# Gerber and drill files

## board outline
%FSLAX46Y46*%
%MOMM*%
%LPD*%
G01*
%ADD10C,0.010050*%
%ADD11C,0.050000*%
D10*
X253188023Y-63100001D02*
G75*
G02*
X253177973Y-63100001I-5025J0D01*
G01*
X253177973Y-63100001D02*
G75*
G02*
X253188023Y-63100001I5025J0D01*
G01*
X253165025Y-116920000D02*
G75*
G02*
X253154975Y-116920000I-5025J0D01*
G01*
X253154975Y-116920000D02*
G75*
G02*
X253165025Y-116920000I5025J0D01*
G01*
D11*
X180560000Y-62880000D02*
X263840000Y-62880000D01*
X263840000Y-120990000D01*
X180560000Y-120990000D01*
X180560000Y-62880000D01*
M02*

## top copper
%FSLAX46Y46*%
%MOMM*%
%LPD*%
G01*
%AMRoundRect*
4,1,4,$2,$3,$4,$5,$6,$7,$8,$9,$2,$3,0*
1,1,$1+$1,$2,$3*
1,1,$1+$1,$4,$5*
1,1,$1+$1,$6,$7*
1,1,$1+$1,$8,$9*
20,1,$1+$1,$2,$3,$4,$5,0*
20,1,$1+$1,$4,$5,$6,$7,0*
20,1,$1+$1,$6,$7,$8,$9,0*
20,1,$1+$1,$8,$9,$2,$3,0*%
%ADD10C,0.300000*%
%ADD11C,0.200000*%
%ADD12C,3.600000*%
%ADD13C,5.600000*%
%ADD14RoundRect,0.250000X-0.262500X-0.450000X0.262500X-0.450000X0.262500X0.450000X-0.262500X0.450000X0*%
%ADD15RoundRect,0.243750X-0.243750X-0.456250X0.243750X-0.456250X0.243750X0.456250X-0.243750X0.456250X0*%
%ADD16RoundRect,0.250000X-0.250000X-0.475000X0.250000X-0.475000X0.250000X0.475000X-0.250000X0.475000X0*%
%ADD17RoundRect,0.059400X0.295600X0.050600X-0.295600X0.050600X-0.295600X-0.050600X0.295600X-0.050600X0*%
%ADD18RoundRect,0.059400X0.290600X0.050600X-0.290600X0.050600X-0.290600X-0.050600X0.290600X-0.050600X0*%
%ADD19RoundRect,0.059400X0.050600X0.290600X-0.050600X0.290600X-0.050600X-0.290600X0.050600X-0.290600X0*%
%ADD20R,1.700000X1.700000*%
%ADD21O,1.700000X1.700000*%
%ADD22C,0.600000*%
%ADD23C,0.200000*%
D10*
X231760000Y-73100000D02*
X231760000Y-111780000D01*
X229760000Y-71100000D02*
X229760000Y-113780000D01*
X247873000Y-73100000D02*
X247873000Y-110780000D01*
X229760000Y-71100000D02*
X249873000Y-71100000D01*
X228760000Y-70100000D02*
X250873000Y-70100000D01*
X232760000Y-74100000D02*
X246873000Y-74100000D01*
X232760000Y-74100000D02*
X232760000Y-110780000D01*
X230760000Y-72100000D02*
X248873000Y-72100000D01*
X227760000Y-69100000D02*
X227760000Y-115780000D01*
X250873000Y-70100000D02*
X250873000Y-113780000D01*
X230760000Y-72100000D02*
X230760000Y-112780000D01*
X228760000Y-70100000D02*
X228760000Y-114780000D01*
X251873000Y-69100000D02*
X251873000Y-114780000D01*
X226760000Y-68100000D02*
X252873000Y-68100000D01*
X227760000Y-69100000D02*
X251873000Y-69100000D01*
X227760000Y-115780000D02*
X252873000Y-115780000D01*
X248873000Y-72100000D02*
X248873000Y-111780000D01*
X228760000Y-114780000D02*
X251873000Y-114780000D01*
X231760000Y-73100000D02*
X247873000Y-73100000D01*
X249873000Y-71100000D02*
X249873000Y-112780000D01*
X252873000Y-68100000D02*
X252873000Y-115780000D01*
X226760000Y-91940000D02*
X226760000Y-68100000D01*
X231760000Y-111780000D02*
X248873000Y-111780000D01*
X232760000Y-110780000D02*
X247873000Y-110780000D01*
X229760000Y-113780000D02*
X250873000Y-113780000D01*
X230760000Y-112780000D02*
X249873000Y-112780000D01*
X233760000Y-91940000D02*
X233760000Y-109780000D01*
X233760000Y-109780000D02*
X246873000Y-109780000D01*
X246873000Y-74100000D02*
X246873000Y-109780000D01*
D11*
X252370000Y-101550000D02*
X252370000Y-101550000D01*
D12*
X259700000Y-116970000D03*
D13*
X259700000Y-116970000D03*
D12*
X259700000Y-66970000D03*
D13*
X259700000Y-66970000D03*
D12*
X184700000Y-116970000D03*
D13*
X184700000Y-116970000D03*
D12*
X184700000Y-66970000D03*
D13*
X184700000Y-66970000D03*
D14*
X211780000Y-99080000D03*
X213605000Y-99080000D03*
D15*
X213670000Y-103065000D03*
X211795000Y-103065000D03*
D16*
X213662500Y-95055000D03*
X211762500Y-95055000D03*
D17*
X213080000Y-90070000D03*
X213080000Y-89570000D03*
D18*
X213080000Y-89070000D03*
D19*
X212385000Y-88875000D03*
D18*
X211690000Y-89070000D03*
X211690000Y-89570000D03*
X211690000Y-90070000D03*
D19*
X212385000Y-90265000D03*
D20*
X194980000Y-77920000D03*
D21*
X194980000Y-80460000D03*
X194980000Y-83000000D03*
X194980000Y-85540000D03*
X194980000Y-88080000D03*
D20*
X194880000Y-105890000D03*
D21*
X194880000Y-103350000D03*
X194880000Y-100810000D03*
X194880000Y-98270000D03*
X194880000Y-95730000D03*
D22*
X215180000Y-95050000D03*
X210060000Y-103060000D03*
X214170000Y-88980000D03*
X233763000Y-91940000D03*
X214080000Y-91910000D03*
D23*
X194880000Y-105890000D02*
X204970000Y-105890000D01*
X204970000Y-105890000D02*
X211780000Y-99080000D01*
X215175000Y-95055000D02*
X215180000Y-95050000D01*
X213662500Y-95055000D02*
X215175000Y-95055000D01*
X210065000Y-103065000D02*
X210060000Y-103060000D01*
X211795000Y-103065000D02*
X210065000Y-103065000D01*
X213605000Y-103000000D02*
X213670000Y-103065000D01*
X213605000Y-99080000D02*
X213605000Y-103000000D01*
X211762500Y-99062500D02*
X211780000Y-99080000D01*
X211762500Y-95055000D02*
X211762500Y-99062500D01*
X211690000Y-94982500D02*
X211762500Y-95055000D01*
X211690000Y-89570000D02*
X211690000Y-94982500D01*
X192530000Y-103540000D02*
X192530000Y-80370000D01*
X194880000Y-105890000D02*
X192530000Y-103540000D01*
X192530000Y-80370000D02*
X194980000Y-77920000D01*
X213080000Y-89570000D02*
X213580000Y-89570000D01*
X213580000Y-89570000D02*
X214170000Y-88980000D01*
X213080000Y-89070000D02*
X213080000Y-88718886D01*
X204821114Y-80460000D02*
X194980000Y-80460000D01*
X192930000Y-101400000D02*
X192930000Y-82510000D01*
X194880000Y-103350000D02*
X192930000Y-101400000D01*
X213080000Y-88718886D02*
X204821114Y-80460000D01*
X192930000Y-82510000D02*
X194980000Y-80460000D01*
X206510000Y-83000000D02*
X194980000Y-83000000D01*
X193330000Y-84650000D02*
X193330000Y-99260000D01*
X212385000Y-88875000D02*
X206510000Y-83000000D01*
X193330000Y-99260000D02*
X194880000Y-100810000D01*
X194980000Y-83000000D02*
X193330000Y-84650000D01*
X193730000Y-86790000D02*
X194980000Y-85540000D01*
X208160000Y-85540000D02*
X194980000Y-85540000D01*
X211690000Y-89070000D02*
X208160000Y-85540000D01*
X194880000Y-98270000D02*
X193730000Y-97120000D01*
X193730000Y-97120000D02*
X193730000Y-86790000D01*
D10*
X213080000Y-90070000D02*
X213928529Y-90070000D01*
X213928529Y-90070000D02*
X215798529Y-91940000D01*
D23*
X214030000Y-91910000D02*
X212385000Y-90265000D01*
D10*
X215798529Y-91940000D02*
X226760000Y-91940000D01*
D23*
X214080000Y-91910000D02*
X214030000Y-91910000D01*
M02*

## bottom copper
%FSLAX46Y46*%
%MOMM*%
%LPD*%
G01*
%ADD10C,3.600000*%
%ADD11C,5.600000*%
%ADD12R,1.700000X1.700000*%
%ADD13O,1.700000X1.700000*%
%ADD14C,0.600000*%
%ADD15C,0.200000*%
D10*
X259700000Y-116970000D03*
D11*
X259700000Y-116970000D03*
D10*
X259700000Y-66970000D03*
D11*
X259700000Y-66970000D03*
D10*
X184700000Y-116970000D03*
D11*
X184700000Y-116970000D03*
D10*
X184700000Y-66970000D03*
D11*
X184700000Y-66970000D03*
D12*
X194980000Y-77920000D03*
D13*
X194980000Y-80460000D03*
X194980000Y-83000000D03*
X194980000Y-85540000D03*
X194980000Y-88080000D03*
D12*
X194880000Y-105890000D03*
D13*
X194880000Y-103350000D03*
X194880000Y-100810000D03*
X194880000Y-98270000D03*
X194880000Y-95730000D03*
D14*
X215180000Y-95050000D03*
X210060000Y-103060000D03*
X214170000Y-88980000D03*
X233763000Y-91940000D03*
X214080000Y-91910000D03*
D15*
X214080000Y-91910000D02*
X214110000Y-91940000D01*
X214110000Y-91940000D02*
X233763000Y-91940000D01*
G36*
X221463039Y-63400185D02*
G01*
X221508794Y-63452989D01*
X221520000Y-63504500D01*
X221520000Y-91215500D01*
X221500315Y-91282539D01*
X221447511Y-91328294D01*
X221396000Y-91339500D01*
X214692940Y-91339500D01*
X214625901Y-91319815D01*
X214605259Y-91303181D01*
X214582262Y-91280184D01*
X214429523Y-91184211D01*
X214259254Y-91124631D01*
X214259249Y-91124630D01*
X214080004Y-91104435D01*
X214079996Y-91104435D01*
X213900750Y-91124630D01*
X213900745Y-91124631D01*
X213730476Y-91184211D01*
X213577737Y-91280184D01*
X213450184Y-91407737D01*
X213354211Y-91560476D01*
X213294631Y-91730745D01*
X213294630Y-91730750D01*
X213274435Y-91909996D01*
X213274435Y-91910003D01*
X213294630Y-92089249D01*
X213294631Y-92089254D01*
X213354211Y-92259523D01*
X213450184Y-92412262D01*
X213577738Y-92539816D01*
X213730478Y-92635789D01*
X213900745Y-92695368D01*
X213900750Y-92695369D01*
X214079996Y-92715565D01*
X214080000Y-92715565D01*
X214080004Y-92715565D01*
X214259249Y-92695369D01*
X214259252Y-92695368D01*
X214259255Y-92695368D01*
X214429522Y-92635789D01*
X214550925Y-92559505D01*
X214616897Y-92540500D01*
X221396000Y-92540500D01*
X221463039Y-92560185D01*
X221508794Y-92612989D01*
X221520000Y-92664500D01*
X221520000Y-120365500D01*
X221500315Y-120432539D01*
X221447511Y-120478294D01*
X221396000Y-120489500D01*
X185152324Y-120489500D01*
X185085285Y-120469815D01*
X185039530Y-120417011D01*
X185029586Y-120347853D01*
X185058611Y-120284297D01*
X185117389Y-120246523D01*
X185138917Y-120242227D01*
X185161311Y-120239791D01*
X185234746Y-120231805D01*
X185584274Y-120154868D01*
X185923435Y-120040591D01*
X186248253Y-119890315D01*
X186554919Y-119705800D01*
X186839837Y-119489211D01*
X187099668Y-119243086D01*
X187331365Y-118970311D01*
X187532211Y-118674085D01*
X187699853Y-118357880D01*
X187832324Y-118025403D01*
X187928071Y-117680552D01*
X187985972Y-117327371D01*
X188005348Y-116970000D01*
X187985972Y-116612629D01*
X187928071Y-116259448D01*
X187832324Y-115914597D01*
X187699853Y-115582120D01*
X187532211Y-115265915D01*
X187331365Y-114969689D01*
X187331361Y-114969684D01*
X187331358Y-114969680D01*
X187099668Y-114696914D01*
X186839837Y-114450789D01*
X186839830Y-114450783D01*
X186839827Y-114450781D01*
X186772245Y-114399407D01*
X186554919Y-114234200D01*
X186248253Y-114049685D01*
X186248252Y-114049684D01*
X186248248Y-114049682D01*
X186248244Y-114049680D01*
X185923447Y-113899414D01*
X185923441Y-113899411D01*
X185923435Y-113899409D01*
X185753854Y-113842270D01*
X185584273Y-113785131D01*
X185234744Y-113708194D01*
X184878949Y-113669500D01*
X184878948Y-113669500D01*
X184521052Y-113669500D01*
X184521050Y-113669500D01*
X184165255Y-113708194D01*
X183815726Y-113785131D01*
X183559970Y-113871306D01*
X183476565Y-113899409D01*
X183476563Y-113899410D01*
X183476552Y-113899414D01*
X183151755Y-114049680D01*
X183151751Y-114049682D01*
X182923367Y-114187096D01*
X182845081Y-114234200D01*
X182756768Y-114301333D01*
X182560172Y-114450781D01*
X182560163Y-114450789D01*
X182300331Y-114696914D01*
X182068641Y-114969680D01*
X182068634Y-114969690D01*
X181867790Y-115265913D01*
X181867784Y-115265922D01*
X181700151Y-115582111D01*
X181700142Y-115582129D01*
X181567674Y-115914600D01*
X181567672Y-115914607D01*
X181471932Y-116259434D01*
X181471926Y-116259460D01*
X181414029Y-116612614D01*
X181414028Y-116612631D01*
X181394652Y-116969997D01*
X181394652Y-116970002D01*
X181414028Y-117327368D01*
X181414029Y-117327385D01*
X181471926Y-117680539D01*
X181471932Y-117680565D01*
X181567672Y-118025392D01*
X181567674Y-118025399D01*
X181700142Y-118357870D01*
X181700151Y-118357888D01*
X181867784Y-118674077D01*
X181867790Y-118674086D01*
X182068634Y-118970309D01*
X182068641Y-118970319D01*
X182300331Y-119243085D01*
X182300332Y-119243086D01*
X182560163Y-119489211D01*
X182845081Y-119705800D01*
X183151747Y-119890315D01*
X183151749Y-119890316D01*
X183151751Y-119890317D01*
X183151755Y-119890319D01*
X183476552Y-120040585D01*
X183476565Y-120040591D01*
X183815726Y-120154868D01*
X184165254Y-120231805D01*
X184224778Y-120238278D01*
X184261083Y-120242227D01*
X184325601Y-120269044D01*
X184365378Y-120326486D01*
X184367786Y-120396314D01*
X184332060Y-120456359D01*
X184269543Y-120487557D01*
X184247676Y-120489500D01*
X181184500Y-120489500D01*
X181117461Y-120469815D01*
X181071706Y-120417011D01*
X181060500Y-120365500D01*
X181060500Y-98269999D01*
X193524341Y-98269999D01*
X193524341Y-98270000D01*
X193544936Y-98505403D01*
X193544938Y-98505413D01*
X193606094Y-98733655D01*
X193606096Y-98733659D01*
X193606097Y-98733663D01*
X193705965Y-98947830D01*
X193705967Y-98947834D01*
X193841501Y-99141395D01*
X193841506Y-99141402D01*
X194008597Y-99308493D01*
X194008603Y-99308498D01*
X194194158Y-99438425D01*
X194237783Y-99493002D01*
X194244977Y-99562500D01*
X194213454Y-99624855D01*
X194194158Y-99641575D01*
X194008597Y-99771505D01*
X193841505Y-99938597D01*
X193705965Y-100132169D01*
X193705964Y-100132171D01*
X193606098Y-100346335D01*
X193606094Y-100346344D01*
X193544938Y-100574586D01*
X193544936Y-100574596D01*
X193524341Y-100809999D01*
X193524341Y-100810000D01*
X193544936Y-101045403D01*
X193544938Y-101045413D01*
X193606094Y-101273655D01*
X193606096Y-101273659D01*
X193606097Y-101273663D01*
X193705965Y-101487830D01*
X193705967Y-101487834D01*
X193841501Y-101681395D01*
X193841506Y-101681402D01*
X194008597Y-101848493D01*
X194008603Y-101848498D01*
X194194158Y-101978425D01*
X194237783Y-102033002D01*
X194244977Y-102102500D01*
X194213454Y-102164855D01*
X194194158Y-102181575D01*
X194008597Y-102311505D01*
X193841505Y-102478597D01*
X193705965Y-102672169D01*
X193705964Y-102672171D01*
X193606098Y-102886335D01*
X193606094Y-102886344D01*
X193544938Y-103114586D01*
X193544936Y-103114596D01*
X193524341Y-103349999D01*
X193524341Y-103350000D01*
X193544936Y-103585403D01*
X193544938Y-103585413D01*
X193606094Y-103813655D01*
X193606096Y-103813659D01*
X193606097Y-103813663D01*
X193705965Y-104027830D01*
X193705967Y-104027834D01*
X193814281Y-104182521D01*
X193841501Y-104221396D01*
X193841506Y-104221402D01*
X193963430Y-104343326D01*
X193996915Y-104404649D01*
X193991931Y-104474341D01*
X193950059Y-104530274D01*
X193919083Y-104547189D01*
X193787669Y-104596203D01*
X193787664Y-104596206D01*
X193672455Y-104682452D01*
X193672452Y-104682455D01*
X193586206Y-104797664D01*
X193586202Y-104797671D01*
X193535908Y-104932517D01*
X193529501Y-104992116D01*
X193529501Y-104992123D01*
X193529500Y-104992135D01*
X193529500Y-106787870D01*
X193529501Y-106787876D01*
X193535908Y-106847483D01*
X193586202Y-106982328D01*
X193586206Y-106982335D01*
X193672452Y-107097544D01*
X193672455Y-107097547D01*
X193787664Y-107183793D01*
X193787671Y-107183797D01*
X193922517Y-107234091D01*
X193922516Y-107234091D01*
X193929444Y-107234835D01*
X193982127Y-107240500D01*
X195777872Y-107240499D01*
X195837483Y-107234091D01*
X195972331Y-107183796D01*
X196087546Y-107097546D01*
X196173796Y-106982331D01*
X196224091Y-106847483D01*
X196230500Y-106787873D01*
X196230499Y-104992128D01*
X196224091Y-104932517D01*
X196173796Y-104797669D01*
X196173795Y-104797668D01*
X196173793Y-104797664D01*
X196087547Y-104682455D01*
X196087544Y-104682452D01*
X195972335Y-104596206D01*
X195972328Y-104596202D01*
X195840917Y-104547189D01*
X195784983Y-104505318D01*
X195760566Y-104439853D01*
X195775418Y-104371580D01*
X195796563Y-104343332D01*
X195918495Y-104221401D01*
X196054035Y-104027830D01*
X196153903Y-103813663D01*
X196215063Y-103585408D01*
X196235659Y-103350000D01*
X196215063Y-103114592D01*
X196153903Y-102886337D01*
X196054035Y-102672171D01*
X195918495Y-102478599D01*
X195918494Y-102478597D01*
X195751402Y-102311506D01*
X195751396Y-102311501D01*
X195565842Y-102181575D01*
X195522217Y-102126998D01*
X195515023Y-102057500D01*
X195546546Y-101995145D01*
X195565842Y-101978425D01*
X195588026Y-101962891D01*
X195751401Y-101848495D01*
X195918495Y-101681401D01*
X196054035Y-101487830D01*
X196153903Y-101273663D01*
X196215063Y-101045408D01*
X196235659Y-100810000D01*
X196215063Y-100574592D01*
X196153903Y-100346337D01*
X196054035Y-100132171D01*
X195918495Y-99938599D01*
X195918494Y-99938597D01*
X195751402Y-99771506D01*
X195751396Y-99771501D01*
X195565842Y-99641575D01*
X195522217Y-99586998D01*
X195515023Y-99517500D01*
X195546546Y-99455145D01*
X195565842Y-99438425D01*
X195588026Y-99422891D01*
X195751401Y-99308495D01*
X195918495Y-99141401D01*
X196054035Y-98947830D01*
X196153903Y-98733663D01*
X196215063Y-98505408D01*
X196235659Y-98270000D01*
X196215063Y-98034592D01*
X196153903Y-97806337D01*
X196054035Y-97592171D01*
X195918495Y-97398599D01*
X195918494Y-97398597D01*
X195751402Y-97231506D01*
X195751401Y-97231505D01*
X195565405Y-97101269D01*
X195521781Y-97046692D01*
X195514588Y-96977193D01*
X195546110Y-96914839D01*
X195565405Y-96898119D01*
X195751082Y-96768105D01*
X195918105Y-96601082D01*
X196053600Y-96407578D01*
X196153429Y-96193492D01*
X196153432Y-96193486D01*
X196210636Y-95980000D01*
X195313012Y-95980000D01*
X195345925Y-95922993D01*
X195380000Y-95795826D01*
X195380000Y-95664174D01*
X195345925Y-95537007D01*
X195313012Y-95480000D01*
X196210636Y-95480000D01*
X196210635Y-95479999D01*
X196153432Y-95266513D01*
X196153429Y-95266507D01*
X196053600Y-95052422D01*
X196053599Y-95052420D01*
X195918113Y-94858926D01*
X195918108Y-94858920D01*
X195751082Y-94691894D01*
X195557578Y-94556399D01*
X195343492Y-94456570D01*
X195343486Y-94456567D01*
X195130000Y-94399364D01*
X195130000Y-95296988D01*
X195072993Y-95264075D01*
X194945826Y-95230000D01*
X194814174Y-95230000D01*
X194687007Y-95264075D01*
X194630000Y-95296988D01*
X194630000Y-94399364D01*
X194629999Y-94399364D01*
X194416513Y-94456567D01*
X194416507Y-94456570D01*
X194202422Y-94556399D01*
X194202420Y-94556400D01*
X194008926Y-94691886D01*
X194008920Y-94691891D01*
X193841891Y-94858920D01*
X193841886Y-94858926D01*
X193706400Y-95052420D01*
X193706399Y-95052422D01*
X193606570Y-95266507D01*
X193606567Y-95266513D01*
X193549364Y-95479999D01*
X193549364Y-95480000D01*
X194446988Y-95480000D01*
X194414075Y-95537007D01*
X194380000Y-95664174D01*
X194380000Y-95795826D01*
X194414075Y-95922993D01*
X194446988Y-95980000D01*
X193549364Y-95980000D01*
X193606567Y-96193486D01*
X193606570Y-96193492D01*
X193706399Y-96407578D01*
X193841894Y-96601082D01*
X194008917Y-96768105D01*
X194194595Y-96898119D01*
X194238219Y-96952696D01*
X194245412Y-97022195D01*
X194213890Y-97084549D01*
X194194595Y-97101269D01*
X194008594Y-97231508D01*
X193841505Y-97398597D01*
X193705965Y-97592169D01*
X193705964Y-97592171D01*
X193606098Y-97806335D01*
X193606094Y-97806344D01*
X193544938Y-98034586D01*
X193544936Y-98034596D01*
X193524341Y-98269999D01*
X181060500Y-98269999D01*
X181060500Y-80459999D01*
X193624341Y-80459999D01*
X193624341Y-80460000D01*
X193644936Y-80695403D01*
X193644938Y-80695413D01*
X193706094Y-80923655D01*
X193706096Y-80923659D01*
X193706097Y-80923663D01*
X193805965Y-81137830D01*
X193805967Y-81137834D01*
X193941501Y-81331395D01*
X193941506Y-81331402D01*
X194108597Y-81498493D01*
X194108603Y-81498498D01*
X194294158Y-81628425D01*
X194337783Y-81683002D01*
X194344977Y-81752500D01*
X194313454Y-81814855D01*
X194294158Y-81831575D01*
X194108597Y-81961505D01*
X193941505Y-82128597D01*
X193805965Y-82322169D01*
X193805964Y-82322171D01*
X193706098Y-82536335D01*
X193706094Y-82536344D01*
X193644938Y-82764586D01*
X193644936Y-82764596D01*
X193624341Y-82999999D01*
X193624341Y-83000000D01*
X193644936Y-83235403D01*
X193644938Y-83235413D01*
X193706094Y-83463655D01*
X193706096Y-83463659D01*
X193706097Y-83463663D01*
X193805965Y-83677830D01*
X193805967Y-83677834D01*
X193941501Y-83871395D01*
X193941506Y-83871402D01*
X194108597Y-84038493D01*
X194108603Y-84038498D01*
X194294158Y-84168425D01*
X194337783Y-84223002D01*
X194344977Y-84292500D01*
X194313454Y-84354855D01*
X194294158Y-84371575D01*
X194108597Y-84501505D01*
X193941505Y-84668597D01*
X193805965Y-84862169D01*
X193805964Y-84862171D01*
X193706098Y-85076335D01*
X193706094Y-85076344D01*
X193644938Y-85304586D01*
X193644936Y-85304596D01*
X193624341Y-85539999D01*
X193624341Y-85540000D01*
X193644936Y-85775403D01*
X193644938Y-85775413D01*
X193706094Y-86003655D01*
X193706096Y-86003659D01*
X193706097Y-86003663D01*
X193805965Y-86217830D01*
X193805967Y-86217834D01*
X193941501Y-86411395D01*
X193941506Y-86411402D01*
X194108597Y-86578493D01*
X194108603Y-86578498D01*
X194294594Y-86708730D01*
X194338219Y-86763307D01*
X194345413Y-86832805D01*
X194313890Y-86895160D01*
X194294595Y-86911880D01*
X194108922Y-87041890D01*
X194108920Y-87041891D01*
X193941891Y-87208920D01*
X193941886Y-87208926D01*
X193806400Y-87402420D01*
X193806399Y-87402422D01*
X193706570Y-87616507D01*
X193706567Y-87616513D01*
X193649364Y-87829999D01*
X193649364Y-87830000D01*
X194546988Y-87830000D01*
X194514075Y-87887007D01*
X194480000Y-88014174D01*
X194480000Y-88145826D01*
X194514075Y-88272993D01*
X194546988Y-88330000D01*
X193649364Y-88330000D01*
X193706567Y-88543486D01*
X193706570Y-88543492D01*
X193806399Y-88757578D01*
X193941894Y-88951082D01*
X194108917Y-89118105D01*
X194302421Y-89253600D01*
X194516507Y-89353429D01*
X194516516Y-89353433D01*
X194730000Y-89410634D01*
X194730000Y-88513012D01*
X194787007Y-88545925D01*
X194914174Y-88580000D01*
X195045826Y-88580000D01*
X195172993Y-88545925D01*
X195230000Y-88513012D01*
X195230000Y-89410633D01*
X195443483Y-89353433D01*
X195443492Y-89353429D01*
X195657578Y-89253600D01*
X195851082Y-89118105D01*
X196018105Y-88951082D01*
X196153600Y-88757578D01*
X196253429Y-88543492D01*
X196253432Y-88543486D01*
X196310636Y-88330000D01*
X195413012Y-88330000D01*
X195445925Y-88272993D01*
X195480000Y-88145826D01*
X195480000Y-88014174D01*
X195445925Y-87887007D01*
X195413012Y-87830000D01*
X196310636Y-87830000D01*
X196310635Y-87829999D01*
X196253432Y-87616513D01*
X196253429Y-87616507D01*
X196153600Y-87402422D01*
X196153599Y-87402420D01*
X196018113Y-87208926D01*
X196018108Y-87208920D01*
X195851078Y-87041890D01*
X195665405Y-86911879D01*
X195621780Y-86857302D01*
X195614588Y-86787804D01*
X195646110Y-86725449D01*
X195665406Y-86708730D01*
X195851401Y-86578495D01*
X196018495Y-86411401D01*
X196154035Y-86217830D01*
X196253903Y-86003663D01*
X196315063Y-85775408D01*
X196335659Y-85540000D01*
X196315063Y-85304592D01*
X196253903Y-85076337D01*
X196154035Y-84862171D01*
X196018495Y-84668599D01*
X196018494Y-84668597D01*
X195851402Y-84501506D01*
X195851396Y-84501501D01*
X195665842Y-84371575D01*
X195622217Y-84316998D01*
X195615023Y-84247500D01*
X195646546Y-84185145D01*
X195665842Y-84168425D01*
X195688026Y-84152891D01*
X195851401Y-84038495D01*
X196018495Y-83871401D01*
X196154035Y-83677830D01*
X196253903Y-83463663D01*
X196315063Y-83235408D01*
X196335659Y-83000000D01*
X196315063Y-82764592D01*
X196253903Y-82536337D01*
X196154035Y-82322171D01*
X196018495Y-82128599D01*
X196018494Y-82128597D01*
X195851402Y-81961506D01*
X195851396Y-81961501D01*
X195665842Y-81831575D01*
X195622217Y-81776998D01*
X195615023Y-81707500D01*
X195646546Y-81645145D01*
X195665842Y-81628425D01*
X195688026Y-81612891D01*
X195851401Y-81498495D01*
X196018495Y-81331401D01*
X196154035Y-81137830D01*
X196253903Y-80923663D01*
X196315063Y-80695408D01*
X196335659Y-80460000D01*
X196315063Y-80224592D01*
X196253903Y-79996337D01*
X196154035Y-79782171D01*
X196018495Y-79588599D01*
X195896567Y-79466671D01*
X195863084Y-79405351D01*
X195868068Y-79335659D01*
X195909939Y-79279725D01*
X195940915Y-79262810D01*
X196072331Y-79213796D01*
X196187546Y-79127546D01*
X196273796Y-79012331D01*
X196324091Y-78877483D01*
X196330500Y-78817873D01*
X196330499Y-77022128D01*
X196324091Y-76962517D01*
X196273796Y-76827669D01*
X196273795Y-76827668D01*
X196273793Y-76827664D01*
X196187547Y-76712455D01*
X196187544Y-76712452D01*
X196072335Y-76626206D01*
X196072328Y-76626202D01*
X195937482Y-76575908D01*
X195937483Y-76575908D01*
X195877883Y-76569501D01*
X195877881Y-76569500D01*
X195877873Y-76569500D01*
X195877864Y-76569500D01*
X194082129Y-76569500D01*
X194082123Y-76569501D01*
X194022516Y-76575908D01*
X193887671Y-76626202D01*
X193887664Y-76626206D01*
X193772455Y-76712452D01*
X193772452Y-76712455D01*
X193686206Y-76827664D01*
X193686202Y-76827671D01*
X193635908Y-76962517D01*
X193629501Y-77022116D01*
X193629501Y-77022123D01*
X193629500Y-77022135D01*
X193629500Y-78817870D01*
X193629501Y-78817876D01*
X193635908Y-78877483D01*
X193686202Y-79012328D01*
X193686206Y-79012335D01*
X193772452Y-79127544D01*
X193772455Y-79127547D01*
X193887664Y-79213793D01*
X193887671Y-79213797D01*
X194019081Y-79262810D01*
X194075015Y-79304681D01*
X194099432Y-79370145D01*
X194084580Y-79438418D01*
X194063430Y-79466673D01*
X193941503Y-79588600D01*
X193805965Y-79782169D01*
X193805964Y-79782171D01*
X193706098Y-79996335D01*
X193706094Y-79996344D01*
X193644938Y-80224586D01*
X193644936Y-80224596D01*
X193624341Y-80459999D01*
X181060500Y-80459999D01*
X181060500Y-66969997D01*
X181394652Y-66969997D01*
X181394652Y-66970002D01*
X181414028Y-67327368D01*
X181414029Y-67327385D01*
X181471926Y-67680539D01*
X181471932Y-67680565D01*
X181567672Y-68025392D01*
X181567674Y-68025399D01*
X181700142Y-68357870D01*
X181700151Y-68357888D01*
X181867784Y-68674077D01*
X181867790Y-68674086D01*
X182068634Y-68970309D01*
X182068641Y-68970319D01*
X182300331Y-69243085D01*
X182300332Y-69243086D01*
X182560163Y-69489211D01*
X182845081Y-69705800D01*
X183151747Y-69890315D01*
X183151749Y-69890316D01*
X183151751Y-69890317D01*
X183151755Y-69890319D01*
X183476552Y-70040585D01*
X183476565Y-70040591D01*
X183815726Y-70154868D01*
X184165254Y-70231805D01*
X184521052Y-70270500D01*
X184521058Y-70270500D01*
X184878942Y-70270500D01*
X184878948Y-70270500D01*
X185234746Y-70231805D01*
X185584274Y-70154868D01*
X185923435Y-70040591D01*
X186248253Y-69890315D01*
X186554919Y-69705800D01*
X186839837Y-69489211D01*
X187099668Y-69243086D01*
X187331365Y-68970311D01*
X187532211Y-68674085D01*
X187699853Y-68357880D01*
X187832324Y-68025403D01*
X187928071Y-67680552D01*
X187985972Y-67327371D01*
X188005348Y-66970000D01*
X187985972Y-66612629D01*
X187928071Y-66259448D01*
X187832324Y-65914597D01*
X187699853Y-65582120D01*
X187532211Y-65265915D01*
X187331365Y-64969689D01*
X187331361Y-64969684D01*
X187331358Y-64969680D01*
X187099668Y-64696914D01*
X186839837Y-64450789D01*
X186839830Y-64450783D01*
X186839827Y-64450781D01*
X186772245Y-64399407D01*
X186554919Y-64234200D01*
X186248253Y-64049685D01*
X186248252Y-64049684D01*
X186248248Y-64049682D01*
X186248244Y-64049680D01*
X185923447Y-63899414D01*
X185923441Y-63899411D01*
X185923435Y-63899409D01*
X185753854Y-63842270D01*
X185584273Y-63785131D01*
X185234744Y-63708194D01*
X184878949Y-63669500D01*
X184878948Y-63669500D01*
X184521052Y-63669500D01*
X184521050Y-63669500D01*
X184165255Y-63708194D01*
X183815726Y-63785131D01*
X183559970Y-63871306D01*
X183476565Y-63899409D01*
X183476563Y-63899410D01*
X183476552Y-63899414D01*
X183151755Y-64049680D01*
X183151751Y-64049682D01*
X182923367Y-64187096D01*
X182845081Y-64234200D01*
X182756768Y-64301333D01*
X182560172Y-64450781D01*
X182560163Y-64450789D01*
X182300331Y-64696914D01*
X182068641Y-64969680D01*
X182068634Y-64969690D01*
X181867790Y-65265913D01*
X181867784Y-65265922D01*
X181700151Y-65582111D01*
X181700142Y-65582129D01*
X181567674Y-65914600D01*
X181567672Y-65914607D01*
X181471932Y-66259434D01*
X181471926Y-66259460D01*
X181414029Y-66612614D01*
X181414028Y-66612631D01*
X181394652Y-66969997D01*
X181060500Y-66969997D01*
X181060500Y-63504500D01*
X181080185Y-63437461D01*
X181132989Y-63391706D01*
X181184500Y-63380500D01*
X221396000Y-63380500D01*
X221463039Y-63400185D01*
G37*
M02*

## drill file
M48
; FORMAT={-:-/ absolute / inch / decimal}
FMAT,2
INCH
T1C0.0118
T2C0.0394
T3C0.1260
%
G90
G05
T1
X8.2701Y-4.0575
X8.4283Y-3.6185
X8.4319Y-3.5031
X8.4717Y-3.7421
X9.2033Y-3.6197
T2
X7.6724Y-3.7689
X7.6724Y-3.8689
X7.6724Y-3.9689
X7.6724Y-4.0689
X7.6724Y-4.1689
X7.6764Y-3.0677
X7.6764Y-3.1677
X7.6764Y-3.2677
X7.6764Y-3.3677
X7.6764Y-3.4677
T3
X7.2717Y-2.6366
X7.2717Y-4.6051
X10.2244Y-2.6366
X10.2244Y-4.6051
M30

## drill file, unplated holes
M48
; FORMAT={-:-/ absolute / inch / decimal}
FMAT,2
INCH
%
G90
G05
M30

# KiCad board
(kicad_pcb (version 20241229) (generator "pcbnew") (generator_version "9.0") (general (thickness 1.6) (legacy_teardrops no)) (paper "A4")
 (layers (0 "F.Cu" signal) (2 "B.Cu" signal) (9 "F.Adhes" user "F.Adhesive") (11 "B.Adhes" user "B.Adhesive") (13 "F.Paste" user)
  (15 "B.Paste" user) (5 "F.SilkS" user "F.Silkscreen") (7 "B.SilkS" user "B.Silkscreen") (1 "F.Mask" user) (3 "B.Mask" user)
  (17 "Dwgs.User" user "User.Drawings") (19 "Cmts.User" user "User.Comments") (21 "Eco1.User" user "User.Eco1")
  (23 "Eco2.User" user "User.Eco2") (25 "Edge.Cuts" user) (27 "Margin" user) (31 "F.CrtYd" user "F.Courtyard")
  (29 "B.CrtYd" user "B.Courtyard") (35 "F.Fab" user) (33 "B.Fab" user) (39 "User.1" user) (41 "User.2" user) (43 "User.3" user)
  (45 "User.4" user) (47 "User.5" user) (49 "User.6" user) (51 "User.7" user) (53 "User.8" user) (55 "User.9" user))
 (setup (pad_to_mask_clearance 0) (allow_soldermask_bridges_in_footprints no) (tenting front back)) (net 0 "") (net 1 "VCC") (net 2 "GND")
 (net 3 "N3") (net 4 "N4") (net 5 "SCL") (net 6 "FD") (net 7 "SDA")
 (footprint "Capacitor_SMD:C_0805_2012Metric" (layer "F.Cu") (at 212.7125 95.055)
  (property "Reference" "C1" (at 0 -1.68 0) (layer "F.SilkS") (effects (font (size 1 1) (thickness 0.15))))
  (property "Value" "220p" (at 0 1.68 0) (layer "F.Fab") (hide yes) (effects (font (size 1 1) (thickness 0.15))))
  (pad "1" smd roundrect (at -0.95 0) (size 1 1.45) (layers "F.Cu" "F.Mask" "F.Paste") (roundrect_rratio 0.25) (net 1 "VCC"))
  (pad "2" smd roundrect (at 0.95 0) (size 1 1.45) (layers "F.Cu" "F.Mask" "F.Paste") (roundrect_rratio 0.25) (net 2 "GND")))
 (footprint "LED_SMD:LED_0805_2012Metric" (layer "F.Cu") (at 212.7325 103.065)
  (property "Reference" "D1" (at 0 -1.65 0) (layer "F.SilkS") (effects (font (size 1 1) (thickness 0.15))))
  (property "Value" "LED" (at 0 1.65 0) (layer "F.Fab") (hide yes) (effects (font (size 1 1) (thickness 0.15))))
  (pad "1" smd roundrect (at -0.9375 0) (size 0.975 1.4) (layers "F.Cu" "F.Mask" "F.Paste") (roundrect_rratio 0.25) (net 2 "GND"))
  (pad "2" smd roundrect (at 0.9375 0) (size 0.975 1.4) (layers "F.Cu" "F.Mask" "F.Paste") (roundrect_rratio 0.25) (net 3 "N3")))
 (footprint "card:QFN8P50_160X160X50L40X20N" (layer "F.Cu") (at 212.385 89.57 180)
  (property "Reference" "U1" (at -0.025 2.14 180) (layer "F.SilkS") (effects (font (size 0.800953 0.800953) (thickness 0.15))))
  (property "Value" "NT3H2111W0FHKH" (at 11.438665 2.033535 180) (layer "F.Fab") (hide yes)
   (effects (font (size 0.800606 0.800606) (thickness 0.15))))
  (pad "1" smd roundrect (at -0.695 -0.5 180) (size 0.71 0.22) (layers "F.Cu" "F.Mask" "F.Paste") (roundrect_rratio 0.27) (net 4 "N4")
   (solder_mask_margin 0.102))
  (pad "2" smd roundrect (at -0.695 0 180) (size 0.71 0.22) (layers "F.Cu" "F.Mask" "F.Paste") (roundrect_rratio 0.27) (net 2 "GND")
   (solder_mask_margin 0.102))
  (pad "3" smd roundrect (at -0.695 0.5 180) (size 0.7 0.22) (layers "F.Cu" "F.Mask" "F.Paste") (roundrect_rratio 0.27) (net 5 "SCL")
   (solder_mask_margin 0.102))
  (pad "4" smd roundrect (at 0 0.695 180) (size 0.22 0.7) (layers "F.Cu" "F.Mask" "F.Paste") (roundrect_rratio 0.27) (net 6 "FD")
   (solder_mask_margin 0.102))
  (pad "5" smd roundrect (at 0.695 0.5 180) (size 0.7 0.22) (layers "F.Cu" "F.Mask" "F.Paste") (roundrect_rratio 0.27) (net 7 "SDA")
   (solder_mask_margin 0.102))
  (pad "6" smd roundrect (at 0.695 0 180) (size 0.7 0.22) (layers "F.Cu" "F.Mask" "F.Paste") (roundrect_rratio 0.27) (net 1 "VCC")
   (solder_mask_margin 0.102))
  (pad "7" smd roundrect (at 0.695 -0.5 180) (size 0.7 0.22) (layers "F.Cu" "F.Mask" "F.Paste") (roundrect_rratio 0.27) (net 1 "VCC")
   (solder_mask_margin 0.102))
  (pad "8" smd roundrect (at 0 -0.695 180) (size 0.22 0.7) (layers "F.Cu" "F.Mask" "F.Paste") (roundrect_rratio 0.27) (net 4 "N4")
   (solder_mask_margin 0.102)))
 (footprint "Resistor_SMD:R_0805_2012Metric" (layer "F.Cu") (at 212.6925 99.08)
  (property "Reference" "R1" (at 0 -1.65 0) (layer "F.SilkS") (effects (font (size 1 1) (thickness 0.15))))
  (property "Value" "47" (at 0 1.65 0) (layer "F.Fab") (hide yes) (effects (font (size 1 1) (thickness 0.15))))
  (pad "1" smd roundrect (at -0.9125 0) (size 1.025 1.4) (layers "F.Cu" "F.Mask" "F.Paste") (roundrect_rratio 0.243902) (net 1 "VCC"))
  (pad "2" smd roundrect (at 0.9125 0) (size 1.025 1.4) (layers "F.Cu" "F.Mask" "F.Paste") (roundrect_rratio 0.243902) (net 3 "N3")))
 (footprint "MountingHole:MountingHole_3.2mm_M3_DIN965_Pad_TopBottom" (layer "F.Cu") (at 259.7 66.97)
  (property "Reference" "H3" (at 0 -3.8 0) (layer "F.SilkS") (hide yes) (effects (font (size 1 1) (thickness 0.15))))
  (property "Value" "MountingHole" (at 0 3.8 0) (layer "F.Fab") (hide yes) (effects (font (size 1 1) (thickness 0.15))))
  (pad "1" thru_hole circle (at 0 0) (size 3.6 3.6) (drill 3.2) (layers "*.Cu" "*.Mask") (remove_unused_layers no))
  (pad "1" connect circle (at 0 0) (size 5.6 5.6) (layers "F.Cu" "F.Mask"))
  (pad "1" connect circle (at 0 0) (size 5.6 5.6) (layers "B.Cu" "B.Mask")))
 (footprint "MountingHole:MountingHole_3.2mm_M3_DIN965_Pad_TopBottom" (layer "F.Cu") (at 184.7 116.97)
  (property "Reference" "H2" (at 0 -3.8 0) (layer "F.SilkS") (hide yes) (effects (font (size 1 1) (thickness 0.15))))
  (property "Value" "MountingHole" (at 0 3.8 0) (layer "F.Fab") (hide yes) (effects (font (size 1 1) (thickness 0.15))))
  (pad "1" thru_hole circle (at 0 0) (size 3.6 3.6) (drill 3.2) (layers "*.Cu" "*.Mask") (remove_unused_layers no))
  (pad "1" connect circle (at 0 0) (size 5.6 5.6) (layers "F.Cu" "F.Mask"))
  (pad "1" connect circle (at 0 0) (size 5.6 5.6) (layers "B.Cu" "B.Mask")))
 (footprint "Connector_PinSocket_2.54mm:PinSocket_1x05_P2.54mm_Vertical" (layer "F.Cu") (at 194.98 77.92)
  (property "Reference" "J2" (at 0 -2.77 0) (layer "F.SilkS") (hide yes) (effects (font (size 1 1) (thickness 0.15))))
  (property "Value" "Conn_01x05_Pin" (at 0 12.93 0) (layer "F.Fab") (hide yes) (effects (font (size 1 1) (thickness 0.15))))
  (pad "1" thru_hole rect (at 0 0) (size 1.7 1.7) (drill 1) (layers "*.Cu" "*.Mask") (remove_unused_layers no) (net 1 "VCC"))
  (pad "2" thru_hole oval (at 0 2.54) (size 1.7 1.7) (drill 1) (layers "*.Cu" "*.Mask") (remove_unused_layers no) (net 5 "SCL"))
  (pad "3" thru_hole oval (at 0 5.08) (size 1.7 1.7) (drill 1) (layers "*.Cu" "*.Mask") (remove_unused_layers no) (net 6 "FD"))
  (pad "4" thru_hole oval (at 0 7.62) (size 1.7 1.7) (drill 1) (layers "*.Cu" "*.Mask") (remove_unused_layers no) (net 7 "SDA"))
  (pad "5" thru_hole oval (at 0 10.16) (size 1.7 1.7) (drill 1) (layers "*.Cu" "*.Mask") (remove_unused_layers no) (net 2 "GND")))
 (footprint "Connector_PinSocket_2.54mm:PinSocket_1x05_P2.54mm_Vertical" (layer "F.Cu") (at 194.88 105.89 180)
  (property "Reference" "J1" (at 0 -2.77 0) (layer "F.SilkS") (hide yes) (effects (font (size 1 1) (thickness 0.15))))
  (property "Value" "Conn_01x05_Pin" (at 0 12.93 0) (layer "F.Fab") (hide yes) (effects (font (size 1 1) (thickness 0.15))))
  (pad "1" thru_hole rect (at 0 0 180) (size 1.7 1.7) (drill 1) (layers "*.Cu" "*.Mask") (remove_unused_layers no) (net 1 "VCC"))
  (pad "2" thru_hole oval (at 0 2.54 180) (size 1.7 1.7) (drill 1) (layers "*.Cu" "*.Mask") (remove_unused_layers no) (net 5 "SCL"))
  (pad "3" thru_hole oval (at 0 5.08 180) (size 1.7 1.7) (drill 1) (layers "*.Cu" "*.Mask") (remove_unused_layers no) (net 6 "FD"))
  (pad "4" thru_hole oval (at 0 7.62 180) (size 1.7 1.7) (drill 1) (layers "*.Cu" "*.Mask") (remove_unused_layers no) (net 7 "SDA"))
  (pad "5" thru_hole oval (at 0 10.16 180) (size 1.7 1.7) (drill 1) (layers "*.Cu" "*.Mask") (remove_unused_layers no) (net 2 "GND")))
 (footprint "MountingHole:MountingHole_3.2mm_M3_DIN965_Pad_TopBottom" (layer "F.Cu") (at 184.7 66.97)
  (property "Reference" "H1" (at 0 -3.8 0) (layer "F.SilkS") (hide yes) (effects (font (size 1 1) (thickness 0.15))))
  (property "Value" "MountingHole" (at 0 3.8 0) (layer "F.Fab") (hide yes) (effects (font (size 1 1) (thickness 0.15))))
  (pad "1" thru_hole circle (at 0 0) (size 3.6 3.6) (drill 3.2) (layers "*.Cu" "*.Mask") (remove_unused_layers no))
  (pad "1" connect circle (at 0 0) (size 5.6 5.6) (layers "F.Cu" "F.Mask"))
  (pad "1" connect circle (at 0 0) (size 5.6 5.6) (layers "B.Cu" "B.Mask")))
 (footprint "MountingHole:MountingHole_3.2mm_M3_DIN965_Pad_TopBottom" (layer "F.Cu") (at 259.7 116.97)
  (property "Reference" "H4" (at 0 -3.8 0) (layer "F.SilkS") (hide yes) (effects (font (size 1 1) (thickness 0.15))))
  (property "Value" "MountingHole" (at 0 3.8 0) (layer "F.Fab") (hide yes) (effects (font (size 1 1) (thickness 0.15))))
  (pad "1" thru_hole circle (at 0 0) (size 3.6 3.6) (drill 3.2) (layers "*.Cu" "*.Mask") (remove_unused_layers no))
  (pad "1" connect circle (at 0 0) (size 5.6 5.6) (layers "F.Cu" "F.Mask"))
  (pad "1" connect circle (at 0 0) (size 5.6 5.6) (layers "B.Cu" "B.Mask")))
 (gr_line (start 231.76 73.1) (end 231.76 111.78) (stroke (width 0.3) (type default)) (layer "F.Cu") (net 4))
 (gr_line (start 229.76 71.1) (end 229.76 113.78) (stroke (width 0.3) (type default)) (layer "F.Cu") (net 4))
 (gr_line (start 247.873 73.1) (end 247.873 110.78) (stroke (width 0.3) (type default)) (layer "F.Cu") (net 4))
 (gr_line (start 229.76 71.1) (end 249.873 71.1) (stroke (width 0.3) (type default)) (layer "F.Cu") (net 4))
 (gr_line (start 228.76 70.1) (end 250.873 70.1) (stroke (width 0.3) (type default)) (layer "F.Cu") (net 4))
 (gr_line (start 232.76 74.1) (end 246.873 74.1) (stroke (width 0.3) (type default)) (layer "F.Cu") (net 4))
 (gr_line (start 232.76 74.1) (end 232.76 110.78) (stroke (width 0.3) (type default)) (layer "F.Cu") (net 4))
 (gr_line (start 230.76 72.1) (end 248.873 72.1) (stroke (width 0.3) (type default)) (layer "F.Cu") (net 4))
 (gr_line (start 227.76 69.1) (end 227.76 115.78) (stroke (width 0.3) (type default)) (layer "F.Cu") (net 4))
 (gr_line (start 250.873 70.1) (end 250.873 113.78) (stroke (width 0.3) (type default)) (layer "F.Cu") (net 4))
 (gr_line (start 230.76 72.1) (end 230.76 112.78) (stroke (width 0.3) (type default)) (layer "F.Cu") (net 4))
 (gr_line (start 228.76 70.1) (end 228.76 114.78) (stroke (width 0.3) (type default)) (layer "F.Cu") (net 4))
 (gr_line (start 251.873 69.1) (end 251.873 114.78) (stroke (width 0.3) (type default)) (layer "F.Cu") (net 4))
 (gr_line (start 226.76 68.1) (end 252.873 68.1) (stroke (width 0.3) (type default)) (layer "F.Cu") (net 4))
 (gr_line (start 227.76 69.1) (end 251.873 69.1) (stroke (width 0.3) (type default)) (layer "F.Cu") (net 4))
 (gr_line (start 227.76 115.78) (end 252.873 115.78) (stroke (width 0.3) (type default)) (layer "F.Cu") (net 4))
 (gr_line (start 248.873 72.1) (end 248.873 111.78) (stroke (width 0.3) (type default)) (layer "F.Cu") (net 4))
 (gr_line (start 228.76 114.78) (end 251.873 114.78) (stroke (width 0.3) (type default)) (layer "F.Cu") (net 4))
 (gr_line (start 231.76 73.1) (end 247.873 73.1) (stroke (width 0.3) (type default)) (layer "F.Cu") (net 4))
 (gr_line (start 249.873 71.1) (end 249.873 112.78) (stroke (width 0.3) (type default)) (layer "F.Cu") (net 4))
 (gr_line (start 252.873 68.1) (end 252.873 115.78) (stroke (width 0.3) (type default)) (layer "F.Cu") (net 4))
 (gr_line (start 226.76 91.94) (end 226.76 68.1) (stroke (width 0.3) (type default)) (layer "F.Cu") (net 4))
 (gr_line (start 231.76 111.78) (end 248.873 111.78) (stroke (width 0.3) (type default)) (layer "F.Cu") (net 4))
 (gr_line (start 232.76 110.78) (end 247.873 110.78) (stroke (width 0.3) (type default)) (layer "F.Cu") (net 4))
 (gr_line (start 229.76 113.78) (end 250.873 113.78) (stroke (width 0.3) (type default)) (layer "F.Cu") (net 4))
 (gr_line (start 230.76 112.78) (end 249.873 112.78) (stroke (width 0.3) (type default)) (layer "F.Cu") (net 4))
 (gr_line (start 233.76 91.94) (end 233.76 109.78) (stroke (width 0.3) (type default)) (layer "F.Cu") (net 4))
 (gr_line (start 233.76 109.78) (end 246.873 109.78) (stroke (width 0.3) (type default)) (layer "F.Cu") (net 4))
 (gr_line (start 246.873 74.1) (end 246.873 109.78) (stroke (width 0.3) (type default)) (layer "F.Cu") (net 4))
 (gr_line (start 252.37 101.55) (end 252.37 101.55) (stroke (width 0.2) (type default)) (layer "F.Cu"))
 (gr_circle (center 253.182998 63.100001) (end 253.192998 63.100001) (stroke (width 0.0001) (type default)) (fill yes) (layer "Edge.Cuts"))
 (gr_circle (center 253.16 116.92) (end 253.17 116.92) (stroke (width 0.0001) (type default)) (fill yes) (layer "Edge.Cuts"))
 (gr_rect (start 180.56 62.88) (end 263.84 120.99) (stroke (width 0.05) (type default)) (fill no) (layer "Edge.Cuts"))
 (segment (start 211.69 89.57) (end 211.69 94.9825) (width 0.2) (layer "F.Cu") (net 1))
 (segment (start 211.7625 99.0625) (end 211.78 99.08) (width 0.2) (layer "F.Cu") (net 1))
 (segment (start 211.69 94.9825) (end 211.7625 95.055) (width 0.2) (layer "F.Cu") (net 1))
 (segment (start 194.88 105.89) (end 204.97 105.89) (width 0.2) (layer "F.Cu") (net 1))
 (segment (start 192.53 103.54) (end 192.53 80.37) (width 0.2) (layer "F.Cu") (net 1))
 (segment (start 194.88 105.89) (end 192.53 103.54) (width 0.2) (layer "F.Cu") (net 1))
 (segment (start 204.97 105.89) (end 211.78 99.08) (width 0.2) (layer "F.Cu") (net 1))
 (segment (start 192.53 80.37) (end 194.98 77.92) (width 0.2) (layer "F.Cu") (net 1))
 (segment (start 211.7625 95.055) (end 211.7625 99.0625) (width 0.2) (layer "F.Cu") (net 1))
 (segment (start 213.6625 95.055) (end 215.175 95.055) (width 0.2) (layer "F.Cu") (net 2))
 (segment (start 213.08 89.57) (end 213.58 89.57) (width 0.2) (layer "F.Cu") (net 2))
 (segment (start 210.065 103.065) (end 210.06 103.06) (width 0.2) (layer "F.Cu") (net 2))
 (segment (start 213.58 89.57) (end 214.17 88.98) (width 0.2) (layer "F.Cu") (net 2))
 (segment (start 211.795 103.065) (end 210.065 103.065) (width 0.2) (layer "F.Cu") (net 2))
 (segment (start 215.175 95.055) (end 215.18 95.05) (width 0.2) (layer "F.Cu") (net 2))
 (via (at 214.17 88.98) (size 0.6) (drill 0.3) (layers "F.Cu" "B.Cu") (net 2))
 (via (at 210.06 103.06) (size 0.6) (drill 0.3) (layers "F.Cu" "B.Cu") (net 2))
 (via (at 215.18 95.05) (size 0.6) (drill 0.3) (layers "F.Cu" "B.Cu") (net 2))
 (segment (start 213.605 103) (end 213.67 103.065) (width 0.2) (layer "F.Cu") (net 3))
 (segment (start 213.605 99.08) (end 213.605 103) (width 0.2) (layer "F.Cu") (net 3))
 (segment (start 213.08 89.07) (end 213.08 88.718886) (width 0.2) (layer "F.Cu") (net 5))
 (segment (start 204.821114 80.46) (end 194.98 80.46) (width 0.2) (layer "F.Cu") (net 5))
 (segment (start 192.93 101.4) (end 192.93 82.51) (width 0.2) (layer "F.Cu") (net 5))
 (segment (start 194.88 103.35) (end 192.93 101.4) (width 0.2) (layer "F.Cu") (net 5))
 (segment (start 213.08 88.718886) (end 204.821114 80.46) (width 0.2) (layer "F.Cu") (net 5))
 (segment (start 192.93 82.51) (end 194.98 80.46) (width 0.2) (layer "F.Cu") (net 5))
 (segment (start 206.51 83) (end 194.98 83) (width 0.2) (layer "F.Cu") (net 6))
 (segment (start 193.33 84.65) (end 193.33 99.26) (width 0.2) (layer "F.Cu") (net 6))
 (segment (start 212.385 88.875) (end 206.51 83) (width 0.2) (layer "F.Cu") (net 6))
 (segment (start 193.33 99.26) (end 194.88 100.81) (width 0.2) (layer "F.Cu") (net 6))
 (segment (start 194.98 83) (end 193.33 84.65) (width 0.2) (layer "F.Cu") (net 6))
 (segment (start 193.73 86.79) (end 194.98 85.54) (width 0.2) (layer "F.Cu") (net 7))
 (segment (start 208.16 85.54) (end 194.98 85.54) (width 0.2) (layer "F.Cu") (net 7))
 (segment (start 211.69 89.07) (end 208.16 85.54) (width 0.2) (layer "F.Cu") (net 7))
 (segment (start 194.88 98.27) (end 193.73 97.12) (width 0.2) (layer "F.Cu") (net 7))
 (segment (start 193.73 97.12) (end 193.73 86.79) (width 0.2) (layer "F.Cu") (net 7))
 (segment (start 213.08 90.07) (end 213.928529 90.07) (width 0.3) (layer "F.Cu") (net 4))
 (segment (start 213.928529 90.07) (end 215.798529 91.94) (width 0.3) (layer "F.Cu") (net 4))
 (segment (start 214.03 91.91) (end 212.385 90.265) (width 0.2) (layer "F.Cu") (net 4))
 (segment (start 215.798529 91.94) (end 226.76 91.94) (width 0.3) (layer "F.Cu") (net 4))
 (segment (start 214.08 91.91) (end 214.03 91.91) (width 0.2) (layer "F.Cu") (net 4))
 (via (at 233.763 91.94) (size 0.6) (drill 0.3) (layers "F.Cu" "B.Cu") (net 4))
 (via (at 214.08 91.91) (size 0.6) (drill 0.3) (layers "F.Cu" "B.Cu") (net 4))
 (segment (start 214.08 91.91) (end 214.11 91.94) (width 0.2) (layer "B.Cu") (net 4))
 (segment (start 214.11 91.94) (end 233.763 91.94) (width 0.2) (layer "B.Cu") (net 4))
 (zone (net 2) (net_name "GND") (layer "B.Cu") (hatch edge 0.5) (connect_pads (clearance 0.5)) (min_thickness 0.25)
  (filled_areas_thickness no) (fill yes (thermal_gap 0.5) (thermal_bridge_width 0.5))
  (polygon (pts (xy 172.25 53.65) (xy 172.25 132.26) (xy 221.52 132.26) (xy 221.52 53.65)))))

